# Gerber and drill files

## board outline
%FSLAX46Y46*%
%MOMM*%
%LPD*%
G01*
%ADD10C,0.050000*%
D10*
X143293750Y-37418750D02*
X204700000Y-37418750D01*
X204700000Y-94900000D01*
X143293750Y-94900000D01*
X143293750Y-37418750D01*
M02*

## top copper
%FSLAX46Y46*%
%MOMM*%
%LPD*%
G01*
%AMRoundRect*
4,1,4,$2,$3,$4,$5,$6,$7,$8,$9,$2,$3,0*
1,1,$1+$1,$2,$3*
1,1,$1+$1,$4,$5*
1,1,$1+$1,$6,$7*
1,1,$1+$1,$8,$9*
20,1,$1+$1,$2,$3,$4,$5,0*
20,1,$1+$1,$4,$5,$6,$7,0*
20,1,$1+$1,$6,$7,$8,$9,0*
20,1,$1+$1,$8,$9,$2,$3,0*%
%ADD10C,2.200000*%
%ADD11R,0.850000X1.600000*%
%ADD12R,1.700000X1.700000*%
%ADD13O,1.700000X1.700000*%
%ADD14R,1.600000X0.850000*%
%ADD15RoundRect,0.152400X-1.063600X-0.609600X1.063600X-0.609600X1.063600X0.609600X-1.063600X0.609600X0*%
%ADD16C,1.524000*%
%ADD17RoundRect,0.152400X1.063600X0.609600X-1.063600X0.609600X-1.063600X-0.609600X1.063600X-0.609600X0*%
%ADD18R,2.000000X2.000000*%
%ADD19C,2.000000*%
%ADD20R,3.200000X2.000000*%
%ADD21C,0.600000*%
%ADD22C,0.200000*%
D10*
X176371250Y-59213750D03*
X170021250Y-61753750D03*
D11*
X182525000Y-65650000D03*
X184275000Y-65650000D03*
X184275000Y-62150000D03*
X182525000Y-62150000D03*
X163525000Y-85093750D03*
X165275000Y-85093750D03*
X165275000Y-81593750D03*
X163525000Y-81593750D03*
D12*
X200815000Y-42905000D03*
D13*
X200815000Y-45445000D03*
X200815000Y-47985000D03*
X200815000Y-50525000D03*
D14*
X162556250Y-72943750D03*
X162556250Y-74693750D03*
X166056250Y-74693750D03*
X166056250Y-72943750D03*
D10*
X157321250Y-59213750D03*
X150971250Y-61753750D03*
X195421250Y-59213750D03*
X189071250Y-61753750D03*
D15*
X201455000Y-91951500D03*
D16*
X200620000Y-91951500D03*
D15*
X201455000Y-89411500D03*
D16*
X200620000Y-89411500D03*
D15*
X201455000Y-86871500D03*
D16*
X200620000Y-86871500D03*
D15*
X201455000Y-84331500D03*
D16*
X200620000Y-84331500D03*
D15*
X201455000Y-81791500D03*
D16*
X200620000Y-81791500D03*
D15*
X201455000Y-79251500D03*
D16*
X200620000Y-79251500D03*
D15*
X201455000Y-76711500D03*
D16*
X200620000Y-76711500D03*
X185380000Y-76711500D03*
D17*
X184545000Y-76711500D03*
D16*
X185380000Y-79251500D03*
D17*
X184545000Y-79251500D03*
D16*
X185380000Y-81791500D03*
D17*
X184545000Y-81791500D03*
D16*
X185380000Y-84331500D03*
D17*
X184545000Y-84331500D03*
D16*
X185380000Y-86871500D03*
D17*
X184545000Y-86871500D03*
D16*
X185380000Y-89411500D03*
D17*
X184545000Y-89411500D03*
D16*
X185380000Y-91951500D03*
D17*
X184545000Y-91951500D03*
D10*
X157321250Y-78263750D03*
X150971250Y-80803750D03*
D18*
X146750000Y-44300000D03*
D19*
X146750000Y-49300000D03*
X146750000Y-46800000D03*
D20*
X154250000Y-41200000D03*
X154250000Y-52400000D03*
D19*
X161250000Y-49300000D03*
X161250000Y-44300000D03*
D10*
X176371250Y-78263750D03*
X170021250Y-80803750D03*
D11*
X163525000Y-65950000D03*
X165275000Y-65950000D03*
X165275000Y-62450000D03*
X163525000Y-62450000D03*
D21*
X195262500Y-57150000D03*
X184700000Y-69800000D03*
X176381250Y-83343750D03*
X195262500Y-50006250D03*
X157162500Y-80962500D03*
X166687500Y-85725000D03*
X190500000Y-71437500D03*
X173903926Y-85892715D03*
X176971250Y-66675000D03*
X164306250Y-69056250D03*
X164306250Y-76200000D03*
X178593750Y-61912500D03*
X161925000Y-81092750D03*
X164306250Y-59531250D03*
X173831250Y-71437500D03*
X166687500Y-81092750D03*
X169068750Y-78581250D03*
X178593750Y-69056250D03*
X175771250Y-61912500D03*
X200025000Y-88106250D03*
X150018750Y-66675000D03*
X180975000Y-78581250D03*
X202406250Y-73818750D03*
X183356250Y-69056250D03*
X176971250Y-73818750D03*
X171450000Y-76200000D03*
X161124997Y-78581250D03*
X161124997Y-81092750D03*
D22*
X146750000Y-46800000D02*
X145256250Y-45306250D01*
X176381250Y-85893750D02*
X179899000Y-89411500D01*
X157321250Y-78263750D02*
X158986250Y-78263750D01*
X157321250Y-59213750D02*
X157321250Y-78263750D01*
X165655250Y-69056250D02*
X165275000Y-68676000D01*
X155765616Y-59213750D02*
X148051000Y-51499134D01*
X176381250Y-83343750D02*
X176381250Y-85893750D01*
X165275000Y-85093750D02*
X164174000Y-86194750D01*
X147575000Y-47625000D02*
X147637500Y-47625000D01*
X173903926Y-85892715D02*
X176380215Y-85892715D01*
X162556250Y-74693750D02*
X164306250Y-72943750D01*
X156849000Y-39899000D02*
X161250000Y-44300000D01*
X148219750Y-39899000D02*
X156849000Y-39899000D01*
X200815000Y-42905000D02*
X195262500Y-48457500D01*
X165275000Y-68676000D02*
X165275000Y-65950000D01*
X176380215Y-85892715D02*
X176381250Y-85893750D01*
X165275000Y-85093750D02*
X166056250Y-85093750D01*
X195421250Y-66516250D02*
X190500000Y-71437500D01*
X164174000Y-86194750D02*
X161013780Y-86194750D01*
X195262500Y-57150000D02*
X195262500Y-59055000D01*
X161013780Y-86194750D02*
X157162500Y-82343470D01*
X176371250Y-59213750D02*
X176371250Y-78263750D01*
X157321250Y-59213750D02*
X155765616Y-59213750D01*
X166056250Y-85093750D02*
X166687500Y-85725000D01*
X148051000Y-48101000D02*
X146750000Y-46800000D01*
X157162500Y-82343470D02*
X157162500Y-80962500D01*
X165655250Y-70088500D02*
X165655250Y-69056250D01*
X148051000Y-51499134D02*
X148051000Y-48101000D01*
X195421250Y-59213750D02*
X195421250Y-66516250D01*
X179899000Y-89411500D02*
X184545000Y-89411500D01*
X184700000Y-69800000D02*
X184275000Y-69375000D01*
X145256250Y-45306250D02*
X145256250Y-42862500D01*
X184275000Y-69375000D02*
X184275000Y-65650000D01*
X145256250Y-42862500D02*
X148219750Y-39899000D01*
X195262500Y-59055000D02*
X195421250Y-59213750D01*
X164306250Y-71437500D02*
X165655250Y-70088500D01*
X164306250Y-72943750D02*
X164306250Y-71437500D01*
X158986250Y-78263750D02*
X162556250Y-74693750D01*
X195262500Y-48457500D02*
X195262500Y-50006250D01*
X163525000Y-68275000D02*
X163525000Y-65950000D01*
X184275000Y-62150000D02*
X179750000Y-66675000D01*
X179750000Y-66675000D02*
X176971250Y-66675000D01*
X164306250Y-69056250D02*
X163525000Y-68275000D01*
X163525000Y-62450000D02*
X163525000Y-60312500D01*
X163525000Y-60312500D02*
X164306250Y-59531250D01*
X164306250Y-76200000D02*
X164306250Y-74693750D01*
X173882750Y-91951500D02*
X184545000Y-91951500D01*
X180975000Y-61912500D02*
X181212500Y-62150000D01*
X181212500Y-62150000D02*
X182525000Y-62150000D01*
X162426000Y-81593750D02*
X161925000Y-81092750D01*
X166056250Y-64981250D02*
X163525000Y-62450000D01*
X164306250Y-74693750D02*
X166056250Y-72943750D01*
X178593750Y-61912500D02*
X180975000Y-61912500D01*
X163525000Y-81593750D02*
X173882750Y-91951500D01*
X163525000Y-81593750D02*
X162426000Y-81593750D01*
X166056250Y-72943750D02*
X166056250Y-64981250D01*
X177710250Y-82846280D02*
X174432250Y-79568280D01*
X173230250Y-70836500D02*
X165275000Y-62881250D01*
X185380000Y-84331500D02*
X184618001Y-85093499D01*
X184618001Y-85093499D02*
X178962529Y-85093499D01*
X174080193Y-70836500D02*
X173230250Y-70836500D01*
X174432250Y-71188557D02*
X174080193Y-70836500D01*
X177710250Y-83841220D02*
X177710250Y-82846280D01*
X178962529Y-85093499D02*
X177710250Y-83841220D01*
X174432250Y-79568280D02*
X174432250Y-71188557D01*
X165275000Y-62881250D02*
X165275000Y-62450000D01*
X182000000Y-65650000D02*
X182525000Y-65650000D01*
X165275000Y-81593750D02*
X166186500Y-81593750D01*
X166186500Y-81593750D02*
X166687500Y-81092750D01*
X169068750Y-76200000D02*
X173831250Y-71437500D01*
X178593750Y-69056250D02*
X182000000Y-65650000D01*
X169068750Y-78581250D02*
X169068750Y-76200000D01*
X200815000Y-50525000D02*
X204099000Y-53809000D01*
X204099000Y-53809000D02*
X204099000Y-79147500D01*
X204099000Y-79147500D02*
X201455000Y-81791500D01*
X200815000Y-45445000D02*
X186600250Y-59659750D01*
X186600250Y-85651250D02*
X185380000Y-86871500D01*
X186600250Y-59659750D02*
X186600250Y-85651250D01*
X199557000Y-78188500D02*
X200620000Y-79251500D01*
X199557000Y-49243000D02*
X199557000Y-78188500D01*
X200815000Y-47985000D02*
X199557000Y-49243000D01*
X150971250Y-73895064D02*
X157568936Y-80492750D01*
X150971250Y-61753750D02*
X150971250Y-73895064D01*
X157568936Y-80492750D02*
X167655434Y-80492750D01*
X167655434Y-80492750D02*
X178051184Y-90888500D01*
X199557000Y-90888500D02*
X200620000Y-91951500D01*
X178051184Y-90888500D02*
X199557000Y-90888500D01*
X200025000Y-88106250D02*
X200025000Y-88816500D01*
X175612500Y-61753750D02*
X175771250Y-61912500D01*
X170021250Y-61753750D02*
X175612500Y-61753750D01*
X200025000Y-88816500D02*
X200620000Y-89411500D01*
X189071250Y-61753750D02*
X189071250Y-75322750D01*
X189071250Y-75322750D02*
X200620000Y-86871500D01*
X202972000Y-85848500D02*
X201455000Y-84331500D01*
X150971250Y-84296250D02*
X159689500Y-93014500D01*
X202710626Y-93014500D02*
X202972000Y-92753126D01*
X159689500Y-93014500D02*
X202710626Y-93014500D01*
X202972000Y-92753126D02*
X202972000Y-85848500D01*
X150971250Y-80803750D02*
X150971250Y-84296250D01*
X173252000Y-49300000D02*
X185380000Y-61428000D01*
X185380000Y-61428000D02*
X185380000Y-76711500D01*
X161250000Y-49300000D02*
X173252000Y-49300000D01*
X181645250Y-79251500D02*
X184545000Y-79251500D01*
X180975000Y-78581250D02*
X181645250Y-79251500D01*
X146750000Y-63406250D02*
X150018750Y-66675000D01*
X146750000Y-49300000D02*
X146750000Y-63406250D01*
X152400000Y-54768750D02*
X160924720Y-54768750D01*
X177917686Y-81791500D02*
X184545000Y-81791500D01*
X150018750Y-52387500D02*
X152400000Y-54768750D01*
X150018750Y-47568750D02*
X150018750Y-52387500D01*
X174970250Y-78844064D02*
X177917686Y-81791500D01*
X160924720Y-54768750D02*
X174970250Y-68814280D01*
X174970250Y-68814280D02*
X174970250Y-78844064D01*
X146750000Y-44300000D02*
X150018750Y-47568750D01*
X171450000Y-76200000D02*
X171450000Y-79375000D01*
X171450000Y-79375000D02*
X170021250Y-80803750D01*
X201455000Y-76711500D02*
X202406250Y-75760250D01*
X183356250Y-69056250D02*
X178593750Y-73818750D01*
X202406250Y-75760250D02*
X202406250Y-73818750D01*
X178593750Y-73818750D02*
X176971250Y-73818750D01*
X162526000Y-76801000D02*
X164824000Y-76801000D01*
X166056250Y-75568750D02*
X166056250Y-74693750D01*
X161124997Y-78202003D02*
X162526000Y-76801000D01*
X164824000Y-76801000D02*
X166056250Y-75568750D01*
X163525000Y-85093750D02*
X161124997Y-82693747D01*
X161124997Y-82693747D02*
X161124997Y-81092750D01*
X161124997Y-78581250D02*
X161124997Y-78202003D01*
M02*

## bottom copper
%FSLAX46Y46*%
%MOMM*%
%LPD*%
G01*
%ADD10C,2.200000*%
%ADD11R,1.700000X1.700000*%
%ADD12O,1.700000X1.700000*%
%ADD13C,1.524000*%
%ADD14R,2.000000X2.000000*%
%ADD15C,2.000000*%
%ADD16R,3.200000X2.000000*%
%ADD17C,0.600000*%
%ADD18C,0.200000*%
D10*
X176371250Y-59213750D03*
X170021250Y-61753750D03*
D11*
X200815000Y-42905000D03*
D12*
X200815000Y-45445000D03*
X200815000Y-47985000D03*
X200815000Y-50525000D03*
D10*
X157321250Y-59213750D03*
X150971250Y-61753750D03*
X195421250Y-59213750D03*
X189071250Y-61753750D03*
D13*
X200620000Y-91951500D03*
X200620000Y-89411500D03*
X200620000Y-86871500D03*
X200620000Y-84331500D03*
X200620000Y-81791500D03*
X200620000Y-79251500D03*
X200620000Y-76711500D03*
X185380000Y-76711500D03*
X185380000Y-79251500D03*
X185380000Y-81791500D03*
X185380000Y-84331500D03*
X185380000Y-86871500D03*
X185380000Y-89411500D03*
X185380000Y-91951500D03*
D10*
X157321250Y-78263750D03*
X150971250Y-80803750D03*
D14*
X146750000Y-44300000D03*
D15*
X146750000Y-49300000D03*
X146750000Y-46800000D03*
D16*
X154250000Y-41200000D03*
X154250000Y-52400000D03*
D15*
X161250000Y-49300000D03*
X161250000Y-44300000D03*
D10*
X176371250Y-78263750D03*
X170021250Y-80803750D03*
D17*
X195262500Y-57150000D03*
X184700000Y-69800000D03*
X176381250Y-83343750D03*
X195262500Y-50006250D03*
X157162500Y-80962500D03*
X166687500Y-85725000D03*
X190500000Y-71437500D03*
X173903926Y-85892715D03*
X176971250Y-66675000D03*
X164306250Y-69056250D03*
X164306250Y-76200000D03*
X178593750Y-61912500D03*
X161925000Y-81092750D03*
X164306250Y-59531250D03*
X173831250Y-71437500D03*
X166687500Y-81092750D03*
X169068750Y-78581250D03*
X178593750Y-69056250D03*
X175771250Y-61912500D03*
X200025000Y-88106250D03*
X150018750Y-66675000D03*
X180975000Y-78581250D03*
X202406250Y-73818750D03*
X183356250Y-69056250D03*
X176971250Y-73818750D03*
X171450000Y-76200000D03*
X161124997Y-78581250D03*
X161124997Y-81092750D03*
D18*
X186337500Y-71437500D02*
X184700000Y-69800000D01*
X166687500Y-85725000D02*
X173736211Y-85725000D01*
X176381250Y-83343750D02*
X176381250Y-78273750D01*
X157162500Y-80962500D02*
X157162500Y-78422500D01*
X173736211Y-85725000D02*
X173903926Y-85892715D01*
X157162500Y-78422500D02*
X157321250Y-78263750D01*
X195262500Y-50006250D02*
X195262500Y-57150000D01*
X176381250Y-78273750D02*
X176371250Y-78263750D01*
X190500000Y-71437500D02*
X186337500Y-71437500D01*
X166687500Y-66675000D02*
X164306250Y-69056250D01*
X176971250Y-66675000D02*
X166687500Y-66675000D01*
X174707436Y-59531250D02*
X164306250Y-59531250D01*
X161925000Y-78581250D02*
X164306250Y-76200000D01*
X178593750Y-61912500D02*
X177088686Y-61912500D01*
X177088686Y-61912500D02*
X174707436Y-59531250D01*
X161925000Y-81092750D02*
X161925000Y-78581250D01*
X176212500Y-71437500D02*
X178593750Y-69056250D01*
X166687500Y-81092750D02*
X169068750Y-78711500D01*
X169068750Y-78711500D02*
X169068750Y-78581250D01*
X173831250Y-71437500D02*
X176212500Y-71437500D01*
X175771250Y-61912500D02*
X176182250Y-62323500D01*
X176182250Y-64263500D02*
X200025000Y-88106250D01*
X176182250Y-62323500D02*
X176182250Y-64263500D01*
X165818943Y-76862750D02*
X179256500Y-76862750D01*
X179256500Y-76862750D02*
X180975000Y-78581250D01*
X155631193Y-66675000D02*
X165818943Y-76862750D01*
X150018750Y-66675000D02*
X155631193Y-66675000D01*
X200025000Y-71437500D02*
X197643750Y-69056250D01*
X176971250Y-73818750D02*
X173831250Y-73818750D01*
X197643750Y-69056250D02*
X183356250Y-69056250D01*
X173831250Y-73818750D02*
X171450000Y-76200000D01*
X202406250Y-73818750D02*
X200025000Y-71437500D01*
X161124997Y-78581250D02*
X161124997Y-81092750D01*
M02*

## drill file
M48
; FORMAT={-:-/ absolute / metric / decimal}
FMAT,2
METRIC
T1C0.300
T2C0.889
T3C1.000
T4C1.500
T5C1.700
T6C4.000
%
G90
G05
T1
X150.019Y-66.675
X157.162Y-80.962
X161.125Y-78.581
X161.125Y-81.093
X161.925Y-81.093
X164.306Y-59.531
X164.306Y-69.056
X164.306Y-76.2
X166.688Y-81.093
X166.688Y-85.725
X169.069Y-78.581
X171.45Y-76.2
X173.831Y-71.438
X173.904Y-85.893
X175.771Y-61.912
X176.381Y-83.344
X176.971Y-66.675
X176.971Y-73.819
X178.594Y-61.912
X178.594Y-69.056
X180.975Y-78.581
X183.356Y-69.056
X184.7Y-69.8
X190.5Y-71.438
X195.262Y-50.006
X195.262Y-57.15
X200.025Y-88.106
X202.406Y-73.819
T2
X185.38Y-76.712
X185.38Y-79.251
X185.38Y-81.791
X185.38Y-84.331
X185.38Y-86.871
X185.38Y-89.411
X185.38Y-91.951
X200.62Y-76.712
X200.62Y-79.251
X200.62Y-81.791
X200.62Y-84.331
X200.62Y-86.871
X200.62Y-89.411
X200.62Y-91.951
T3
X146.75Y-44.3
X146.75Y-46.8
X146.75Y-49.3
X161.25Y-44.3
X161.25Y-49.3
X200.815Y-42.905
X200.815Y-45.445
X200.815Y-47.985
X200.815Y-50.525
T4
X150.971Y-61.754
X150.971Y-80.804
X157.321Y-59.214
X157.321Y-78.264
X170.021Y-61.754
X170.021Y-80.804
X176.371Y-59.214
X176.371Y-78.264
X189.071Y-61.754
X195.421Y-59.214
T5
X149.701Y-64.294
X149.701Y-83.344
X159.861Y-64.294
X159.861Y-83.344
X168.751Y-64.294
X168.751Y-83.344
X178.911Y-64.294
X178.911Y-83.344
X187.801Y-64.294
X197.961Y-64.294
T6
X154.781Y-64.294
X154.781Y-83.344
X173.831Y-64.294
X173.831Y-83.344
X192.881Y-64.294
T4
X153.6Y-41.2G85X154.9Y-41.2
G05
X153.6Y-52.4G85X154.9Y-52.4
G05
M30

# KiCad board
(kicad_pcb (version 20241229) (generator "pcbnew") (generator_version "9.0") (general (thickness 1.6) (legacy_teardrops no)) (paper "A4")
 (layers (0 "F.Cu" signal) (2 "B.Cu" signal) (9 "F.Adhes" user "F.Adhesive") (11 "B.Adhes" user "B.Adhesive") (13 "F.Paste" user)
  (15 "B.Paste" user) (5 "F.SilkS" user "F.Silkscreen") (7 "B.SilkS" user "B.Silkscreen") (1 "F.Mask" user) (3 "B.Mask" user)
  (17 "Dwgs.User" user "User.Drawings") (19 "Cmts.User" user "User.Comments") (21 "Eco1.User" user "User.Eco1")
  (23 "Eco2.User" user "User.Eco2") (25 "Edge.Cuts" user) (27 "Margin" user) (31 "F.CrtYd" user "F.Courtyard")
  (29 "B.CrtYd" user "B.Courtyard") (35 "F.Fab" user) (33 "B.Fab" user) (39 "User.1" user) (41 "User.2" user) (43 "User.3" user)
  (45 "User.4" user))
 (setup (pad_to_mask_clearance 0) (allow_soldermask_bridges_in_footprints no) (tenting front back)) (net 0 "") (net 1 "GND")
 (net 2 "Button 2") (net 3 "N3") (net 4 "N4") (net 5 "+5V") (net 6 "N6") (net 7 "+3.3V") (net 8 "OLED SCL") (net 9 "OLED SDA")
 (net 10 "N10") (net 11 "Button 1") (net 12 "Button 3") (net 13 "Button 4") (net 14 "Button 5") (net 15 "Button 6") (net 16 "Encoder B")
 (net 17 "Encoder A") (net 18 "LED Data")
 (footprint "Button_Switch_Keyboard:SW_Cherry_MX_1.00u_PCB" (layer "F.Cu") (at 176.37125 59.21375)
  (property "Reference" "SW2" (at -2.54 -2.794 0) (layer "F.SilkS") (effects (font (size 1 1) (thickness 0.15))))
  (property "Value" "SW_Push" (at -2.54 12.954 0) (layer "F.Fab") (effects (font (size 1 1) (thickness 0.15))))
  (pad "" np_thru_hole circle (at -7.62 5.08) (size 1.7 1.7) (drill 1.7) (layers "*.Cu" "*.Mask"))
  (pad "" np_thru_hole circle (at -2.54 5.08) (size 4 4) (drill 4) (layers "*.Cu" "*.Mask"))
  (pad "" np_thru_hole circle (at 2.54 5.08) (size 1.7 1.7) (drill 1.7) (layers "*.Cu" "*.Mask"))
  (pad "1" thru_hole circle (at 0 0) (size 2.2 2.2) (drill 1.5) (layers "*.Cu" "*.Mask") (remove_unused_layers no) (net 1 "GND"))
  (pad "2" thru_hole circle (at -6.35 2.54) (size 2.2 2.2) (drill 1.5) (layers "*.Cu" "*.Mask") (remove_unused_layers no) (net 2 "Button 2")))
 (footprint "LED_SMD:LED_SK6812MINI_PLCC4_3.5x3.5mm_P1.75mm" (layer "F.Cu") (at 183.4 63.9 90)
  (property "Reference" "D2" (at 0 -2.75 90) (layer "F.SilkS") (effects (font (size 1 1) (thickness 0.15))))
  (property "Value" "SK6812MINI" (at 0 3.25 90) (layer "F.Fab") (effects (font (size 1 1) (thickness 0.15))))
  (pad "1" smd rect (at -1.75 -0.875 90) (size 1.6 0.85) (layers "F.Cu" "F.Mask" "F.Paste") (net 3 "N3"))
  (pad "2" smd rect (at -1.75 0.875 90) (size 1.6 0.85) (layers "F.Cu" "F.Mask" "F.Paste") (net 1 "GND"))
  (pad "3" smd rect (at 1.75 0.875 90) (size 1.6 0.85) (layers "F.Cu" "F.Mask" "F.Paste") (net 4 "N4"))
  (pad "4" smd rect (at 1.75 -0.875 90) (size 1.6 0.85) (layers "F.Cu" "F.Mask" "F.Paste") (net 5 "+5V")))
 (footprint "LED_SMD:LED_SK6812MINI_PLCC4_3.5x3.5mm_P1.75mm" (layer "F.Cu") (at 164.4 83.34375 90)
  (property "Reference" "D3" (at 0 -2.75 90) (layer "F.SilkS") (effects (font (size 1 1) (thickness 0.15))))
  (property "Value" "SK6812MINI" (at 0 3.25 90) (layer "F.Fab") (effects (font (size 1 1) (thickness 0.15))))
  (pad "1" smd rect (at -1.75 -0.875 90) (size 1.6 0.85) (layers "F.Cu" "F.Mask" "F.Paste") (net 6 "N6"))
  (pad "2" smd rect (at -1.75 0.875 90) (size 1.6 0.85) (layers "F.Cu" "F.Mask" "F.Paste") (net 1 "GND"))
  (pad "3" smd rect (at 1.75 0.875 90) (size 1.6 0.85) (layers "F.Cu" "F.Mask" "F.Paste") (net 3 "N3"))
  (pad "4" smd rect (at 1.75 -0.875 90) (size 1.6 0.85) (layers "F.Cu" "F.Mask" "F.Paste") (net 5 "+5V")))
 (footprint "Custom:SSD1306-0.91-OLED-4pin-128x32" (layer "F.Cu") (at 164.315 40.715)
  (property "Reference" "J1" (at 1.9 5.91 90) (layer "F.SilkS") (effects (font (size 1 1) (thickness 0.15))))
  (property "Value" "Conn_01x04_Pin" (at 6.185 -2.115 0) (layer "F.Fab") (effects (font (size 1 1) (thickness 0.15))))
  (pad "1" thru_hole rect (at 36.5 2.19) (size 1.7 1.7) (drill 1) (layers "*.Cu" "*.Mask") (remove_unused_layers no) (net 1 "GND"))
  (pad "2" thru_hole oval (at 36.5 4.73) (size 1.7 1.7) (drill 1) (layers "*.Cu" "*.Mask") (remove_unused_layers no) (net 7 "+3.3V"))
  (pad "3" thru_hole oval (at 36.5 7.27) (size 1.7 1.7) (drill 1) (layers "*.Cu" "*.Mask") (remove_unused_layers no) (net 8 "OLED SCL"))
  (pad "4" thru_hole oval (at 36.5 9.81) (size 1.7 1.7) (drill 1) (layers "*.Cu" "*.Mask") (remove_unused_layers no) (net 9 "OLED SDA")))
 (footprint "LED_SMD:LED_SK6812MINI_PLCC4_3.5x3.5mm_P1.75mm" (layer "F.Cu") (at 164.30625 73.81875)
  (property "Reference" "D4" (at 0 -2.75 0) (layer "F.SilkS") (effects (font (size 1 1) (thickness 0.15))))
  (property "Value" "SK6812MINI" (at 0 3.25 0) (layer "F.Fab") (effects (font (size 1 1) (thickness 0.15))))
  (pad "1" smd rect (at -1.75 -0.875) (size 1.6 0.85) (layers "F.Cu" "F.Mask" "F.Paste") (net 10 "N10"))
  (pad "2" smd rect (at -1.75 0.875) (size 1.6 0.85) (layers "F.Cu" "F.Mask" "F.Paste") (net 1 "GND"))
  (pad "3" smd rect (at 1.75 0.875) (size 1.6 0.85) (layers "F.Cu" "F.Mask" "F.Paste") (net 6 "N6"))
  (pad "4" smd rect (at 1.75 -0.875) (size 1.6 0.85) (layers "F.Cu" "F.Mask" "F.Paste") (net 5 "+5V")))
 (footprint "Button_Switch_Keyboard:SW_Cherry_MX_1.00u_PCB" (layer "F.Cu") (at 157.32125 59.21375)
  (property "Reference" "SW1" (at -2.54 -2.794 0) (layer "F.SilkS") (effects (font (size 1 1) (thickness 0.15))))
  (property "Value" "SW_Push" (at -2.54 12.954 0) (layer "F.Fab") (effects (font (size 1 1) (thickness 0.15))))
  (pad "" np_thru_hole circle (at -7.62 5.08) (size 1.7 1.7) (drill 1.7) (layers "*.Cu" "*.Mask"))
  (pad "" np_thru_hole circle (at -2.54 5.08) (size 4 4) (drill 4) (layers "*.Cu" "*.Mask"))
  (pad "" np_thru_hole circle (at 2.54 5.08) (size 1.7 1.7) (drill 1.7) (layers "*.Cu" "*.Mask"))
  (pad "1" thru_hole circle (at 0 0) (size 2.2 2.2) (drill 1.5) (layers "*.Cu" "*.Mask") (remove_unused_layers no) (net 1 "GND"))
  (pad "2" thru_hole circle (at -6.35 2.54) (size 2.2 2.2) (drill 1.5) (layers "*.Cu" "*.Mask") (remove_unused_layers no)
   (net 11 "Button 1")))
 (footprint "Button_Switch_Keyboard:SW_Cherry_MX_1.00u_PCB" (layer "F.Cu") (at 195.42125 59.21375)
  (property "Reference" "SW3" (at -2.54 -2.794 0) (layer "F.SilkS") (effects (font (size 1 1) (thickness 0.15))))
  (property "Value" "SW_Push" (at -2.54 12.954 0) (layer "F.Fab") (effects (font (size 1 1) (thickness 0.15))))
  (pad "" np_thru_hole circle (at -7.62 5.08) (size 1.7 1.7) (drill 1.7) (layers "*.Cu" "*.Mask"))
  (pad "" np_thru_hole circle (at -2.54 5.08) (size 4 4) (drill 4) (layers "*.Cu" "*.Mask"))
  (pad "" np_thru_hole circle (at 2.54 5.08) (size 1.7 1.7) (drill 1.7) (layers "*.Cu" "*.Mask"))
  (pad "1" thru_hole circle (at 0 0) (size 2.2 2.2) (drill 1.5) (layers "*.Cu" "*.Mask") (remove_unused_layers no) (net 1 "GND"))
  (pad "2" thru_hole circle (at -6.35 2.54) (size 2.2 2.2) (drill 1.5) (layers "*.Cu" "*.Mask") (remove_unused_layers no)
   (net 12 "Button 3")))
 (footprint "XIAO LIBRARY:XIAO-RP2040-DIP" (layer "F.Cu") (at 193 84.3315 180)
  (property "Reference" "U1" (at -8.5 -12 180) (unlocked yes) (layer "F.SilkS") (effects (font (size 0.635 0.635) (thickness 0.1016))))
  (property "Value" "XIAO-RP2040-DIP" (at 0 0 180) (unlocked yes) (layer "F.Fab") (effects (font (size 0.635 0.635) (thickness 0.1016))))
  (pad "1" smd roundrect (at -8.455 -7.62) (size 2.432 1.524) (layers "F.Cu" "F.Mask") (roundrect_rratio 0.1) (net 11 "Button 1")
   (thermal_bridge_angle 45))
  (pad "1" thru_hole circle (at -7.62 -7.62) (size 1.524 1.524) (drill 0.889) (layers "*.Cu" "*.Mask") (remove_unused_layers no)
   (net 11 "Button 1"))
  (pad "2" smd roundrect (at -8.455 -5.08) (size 2.432 1.524) (layers "F.Cu" "F.Mask") (roundrect_rratio 0.1) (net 2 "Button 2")
   (thermal_bridge_angle 45))
  (pad "2" thru_hole circle (at -7.62 -5.08) (size 1.524 1.524) (drill 0.889) (layers "*.Cu" "*.Mask") (remove_unused_layers no)
   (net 2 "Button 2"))
  (pad "3" smd roundrect (at -8.455 -2.54) (size 2.432 1.524) (layers "F.Cu" "F.Mask") (roundrect_rratio 0.1) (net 12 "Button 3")
   (thermal_bridge_angle 45))
  (pad "3" thru_hole circle (at -7.62 -2.54) (size 1.524 1.524) (drill 0.889) (layers "*.Cu" "*.Mask") (remove_unused_layers no)
   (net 12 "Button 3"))
  (pad "4" smd roundrect (at -8.455 0) (size 2.432 1.524) (layers "F.Cu" "F.Mask") (roundrect_rratio 0.1) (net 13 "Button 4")
   (thermal_bridge_angle 45))
  (pad "4" thru_hole circle (at -7.62 0) (size 1.524 1.524) (drill 0.889) (layers "*.Cu" "*.Mask") (remove_unused_layers no)
   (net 13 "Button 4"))
  (pad "5" smd roundrect (at -8.455 2.54) (size 2.432 1.524) (layers "F.Cu" "F.Mask") (roundrect_rratio 0.1) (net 9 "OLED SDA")
   (thermal_bridge_angle 45))
  (pad "5" thru_hole circle (at -7.62 2.54) (size 1.524 1.524) (drill 0.889) (layers "*.Cu" "*.Mask") (remove_unused_layers no)
   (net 9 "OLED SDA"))
  (pad "6" smd roundrect (at -8.455 5.08) (size 2.432 1.524) (layers "F.Cu" "F.Mask") (roundrect_rratio 0.1) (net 8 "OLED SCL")
   (thermal_bridge_angle 45))
  (pad "6" thru_hole circle (at -7.62 5.08) (size 1.524 1.524) (drill 0.889) (layers "*.Cu" "*.Mask") (remove_unused_layers no)
   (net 8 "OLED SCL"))
  (pad "7" smd roundrect (at -8.455 7.62) (size 2.432 1.524) (layers "F.Cu" "F.Mask") (roundrect_rratio 0.1) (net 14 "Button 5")
   (thermal_bridge_angle 45))
  (pad "7" thru_hole circle (at -7.62 7.62) (size 1.524 1.524) (drill 0.889) (layers "*.Cu" "*.Mask") (remove_unused_layers no)
   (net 14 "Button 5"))
  (pad "8" thru_hole circle (at 7.62 7.62 180) (size 1.524 1.524) (drill 0.889) (layers "*.Cu" "*.Mask") (remove_unused_layers no)
   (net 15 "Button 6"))
  (pad "8" smd roundrect (at 8.455 7.62 180) (size 2.432 1.524) (layers "F.Cu" "F.Mask") (roundrect_rratio 0.1) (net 15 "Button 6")
   (thermal_bridge_angle 45))
  (pad "9" thru_hole circle (at 7.62 5.08 180) (size 1.524 1.524) (drill 0.889) (layers "*.Cu" "*.Mask") (remove_unused_layers no)
   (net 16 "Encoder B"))
  (pad "9" smd roundrect (at 8.455 5.08 180) (size 2.432 1.524) (layers "F.Cu" "F.Mask") (roundrect_rratio 0.1) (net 16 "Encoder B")
   (thermal_bridge_angle 45))
  (pad "10" thru_hole circle (at 7.62 2.54 180) (size 1.524 1.524) (drill 0.889) (layers "*.Cu" "*.Mask") (remove_unused_layers no)
   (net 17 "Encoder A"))
  (pad "10" smd roundrect (at 8.455 2.54 180) (size 2.432 1.524) (layers "F.Cu" "F.Mask") (roundrect_rratio 0.1) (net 17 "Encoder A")
   (thermal_bridge_angle 45))
  (pad "11" thru_hole circle (at 7.62 0 180) (size 1.524 1.524) (drill 0.889) (layers "*.Cu" "*.Mask") (remove_unused_layers no)
   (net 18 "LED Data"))
  (pad "11" smd roundrect (at 8.455 0 180) (size 2.432 1.524) (layers "F.Cu" "F.Mask") (roundrect_rratio 0.1) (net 18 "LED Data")
   (thermal_bridge_angle 45))
  (pad "12" thru_hole circle (at 7.62 -2.54 180) (size 1.524 1.524) (drill 0.889) (layers "*.Cu" "*.Mask") (remove_unused_layers no)
   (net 7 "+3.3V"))
  (pad "12" smd roundrect (at 8.455 -2.54 180) (size 2.432 1.524) (layers "F.Cu" "F.Mask") (roundrect_rratio 0.1) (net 7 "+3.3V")
   (thermal_bridge_angle 45))
  (pad "13" thru_hole circle (at 7.62 -5.08 180) (size 1.524 1.524) (drill 0.889) (layers "*.Cu" "*.Mask") (remove_unused_layers no)
   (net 1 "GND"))
  (pad "13" smd roundrect (at 8.455 -5.08 180) (size 2.432 1.524) (layers "F.Cu" "F.Mask") (roundrect_rratio 0.1) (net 1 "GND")
   (thermal_bridge_angle 45))
  (pad "14" thru_hole circle (at 7.62 -7.62 180) (size 1.524 1.524) (drill 0.889) (layers "*.Cu" "*.Mask") (remove_unused_layers no)
   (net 5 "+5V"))
  (pad "14" smd roundrect (at 8.455 -7.62 180) (size 2.432 1.524) (layers "F.Cu" "F.Mask") (roundrect_rratio 0.1) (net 5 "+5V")
   (thermal_bridge_angle 45)))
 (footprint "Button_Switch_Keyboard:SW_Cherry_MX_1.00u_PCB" (layer "F.Cu") (at 157.32125 78.26375)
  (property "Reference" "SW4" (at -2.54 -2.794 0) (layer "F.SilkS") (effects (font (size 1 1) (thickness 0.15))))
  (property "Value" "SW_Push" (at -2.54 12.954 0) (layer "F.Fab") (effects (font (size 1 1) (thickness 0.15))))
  (pad "" np_thru_hole circle (at -7.62 5.08) (size 1.7 1.7) (drill 1.7) (layers "*.Cu" "*.Mask"))
  (pad "" np_thru_hole circle (at -2.54 5.08) (size 4 4) (drill 4) (layers "*.Cu" "*.Mask"))
  (pad "" np_thru_hole circle (at 2.54 5.08) (size 1.7 1.7) (drill 1.7) (layers "*.Cu" "*.Mask"))
  (pad "1" thru_hole circle (at 0 0) (size 2.2 2.2) (drill 1.5) (layers "*.Cu" "*.Mask") (remove_unused_layers no) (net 1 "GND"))
  (pad "2" thru_hole circle (at -6.35 2.54) (size 2.2 2.2) (drill 1.5) (layers "*.Cu" "*.Mask") (remove_unused_layers no)
   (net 13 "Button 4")))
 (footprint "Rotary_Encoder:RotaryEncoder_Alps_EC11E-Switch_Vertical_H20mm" (layer "F.Cu") (at 146.75 44.3)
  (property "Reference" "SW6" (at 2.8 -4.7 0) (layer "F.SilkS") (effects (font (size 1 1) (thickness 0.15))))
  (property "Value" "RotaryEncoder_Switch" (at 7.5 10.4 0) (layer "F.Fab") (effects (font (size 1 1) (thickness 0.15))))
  (pad "A" thru_hole rect (at 0 0) (size 2 2) (drill 1) (layers "*.Cu" "*.Mask") (remove_unused_layers no) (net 17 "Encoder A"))
  (pad "B" thru_hole circle (at 0 5) (size 2 2) (drill 1) (layers "*.Cu" "*.Mask") (remove_unused_layers no) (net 16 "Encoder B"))
  (pad "C" thru_hole circle (at 0 2.5) (size 2 2) (drill 1) (layers "*.Cu" "*.Mask") (remove_unused_layers no) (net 1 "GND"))
  (pad "MP" thru_hole rect (at 7.5 -3.1) (size 3.2 2) (drill oval 2.8 1.5) (layers "*.Cu" "*.Mask") (remove_unused_layers no))
  (pad "MP" thru_hole rect (at 7.5 8.1) (size 3.2 2) (drill oval 2.8 1.5) (layers "*.Cu" "*.Mask") (remove_unused_layers no))
  (pad "S1" thru_hole circle (at 14.5 5) (size 2 2) (drill 1) (layers "*.Cu" "*.Mask") (remove_unused_layers no) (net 15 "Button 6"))
  (pad "S2" thru_hole circle (at 14.5 0) (size 2 2) (drill 1) (layers "*.Cu" "*.Mask") (remove_unused_layers no) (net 1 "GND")))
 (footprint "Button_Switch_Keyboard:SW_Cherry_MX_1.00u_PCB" (layer "F.Cu") (at 176.37125 78.26375)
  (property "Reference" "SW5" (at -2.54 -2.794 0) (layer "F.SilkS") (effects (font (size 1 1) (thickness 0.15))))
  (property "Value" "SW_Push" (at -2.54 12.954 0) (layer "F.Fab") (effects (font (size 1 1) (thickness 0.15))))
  (pad "" np_thru_hole circle (at -7.62 5.08) (size 1.7 1.7) (drill 1.7) (layers "*.Cu" "*.Mask"))
  (pad "" np_thru_hole circle (at -2.54 5.08) (size 4 4) (drill 4) (layers "*.Cu" "*.Mask"))
  (pad "" np_thru_hole circle (at 2.54 5.08) (size 1.7 1.7) (drill 1.7) (layers "*.Cu" "*.Mask"))
  (pad "1" thru_hole circle (at 0 0) (size 2.2 2.2) (drill 1.5) (layers "*.Cu" "*.Mask") (remove_unused_layers no) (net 1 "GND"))
  (pad "2" thru_hole circle (at -6.35 2.54) (size 2.2 2.2) (drill 1.5) (layers "*.Cu" "*.Mask") (remove_unused_layers no)
   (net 14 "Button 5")))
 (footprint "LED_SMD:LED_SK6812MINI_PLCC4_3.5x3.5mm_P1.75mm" (layer "F.Cu") (at 164.4 64.2 90)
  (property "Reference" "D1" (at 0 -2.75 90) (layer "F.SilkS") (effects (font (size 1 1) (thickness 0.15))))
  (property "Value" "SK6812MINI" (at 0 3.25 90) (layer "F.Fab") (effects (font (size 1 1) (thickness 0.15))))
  (pad "1" smd rect (at -1.75 -0.875 90) (size 1.6 0.85) (layers "F.Cu" "F.Mask" "F.Paste") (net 4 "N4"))
  (pad "2" smd rect (at -1.75 0.875 90) (size 1.6 0.85) (layers "F.Cu" "F.Mask" "F.Paste") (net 1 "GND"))
  (pad "3" smd rect (at 1.75 0.875 90) (size 1.6 0.85) (layers "F.Cu" "F.Mask" "F.Paste") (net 18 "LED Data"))
  (pad "4" smd rect (at 1.75 -0.875 90) (size 1.6 0.85) (layers "F.Cu" "F.Mask" "F.Paste") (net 5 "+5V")))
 (gr_rect (start 143.29375 37.41875) (end 204.7 94.9) (stroke (width 0.05) (type default)) (fill no) (layer "Edge.Cuts"))
 (segment (start 146.75 46.8) (end 145.25625 45.30625) (width 0.2) (layer "F.Cu") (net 1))
 (segment (start 176.38125 85.89375) (end 179.899 89.4115) (width 0.2) (layer "F.Cu") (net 1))
 (segment (start 157.32125 78.26375) (end 158.98625 78.26375) (width 0.2) (layer "F.Cu") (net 1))
 (segment (start 157.32125 59.21375) (end 157.32125 78.26375) (width 0.2) (layer "F.Cu") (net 1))
 (segment (start 165.65525 69.05625) (end 165.275 68.676) (width 0.2) (layer "F.Cu") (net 1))
 (segment (start 155.765616 59.21375) (end 148.051 51.499134) (width 0.2) (layer "F.Cu") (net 1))
 (segment (start 176.38125 83.34375) (end 176.38125 85.89375) (width 0.2) (layer "F.Cu") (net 1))
 (segment (start 165.275 85.09375) (end 164.174 86.19475) (width 0.2) (layer "F.Cu") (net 1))
 (segment (start 147.575 47.625) (end 147.6375 47.625) (width 0.2) (layer "F.Cu") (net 1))
 (segment (start 173.903926 85.892715) (end 176.380215 85.892715) (width 0.2) (layer "F.Cu") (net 1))
 (segment (start 162.55625 74.69375) (end 164.30625 72.94375) (width 0.2) (layer "F.Cu") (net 1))
 (segment (start 156.849 39.899) (end 161.25 44.3) (width 0.2) (layer "F.Cu") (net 1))
 (segment (start 148.21975 39.899) (end 156.849 39.899) (width 0.2) (layer "F.Cu") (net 1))
 (segment (start 200.815 42.905) (end 195.2625 48.4575) (width 0.2) (layer "F.Cu") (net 1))
 (segment (start 165.275 68.676) (end 165.275 65.95) (width 0.2) (layer "F.Cu") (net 1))
 (segment (start 176.380215 85.892715) (end 176.38125 85.89375) (width 0.2) (layer "F.Cu") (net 1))
 (segment (start 165.275 85.09375) (end 166.05625 85.09375) (width 0.2) (layer "F.Cu") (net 1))
 (segment (start 195.42125 66.51625) (end 190.5 71.4375) (width 0.2) (layer "F.Cu") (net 1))
 (segment (start 164.174 86.19475) (end 161.01378 86.19475) (width 0.2) (layer "F.Cu") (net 1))
 (segment (start 195.2625 57.15) (end 195.2625 59.055) (width 0.2) (layer "F.Cu") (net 1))
 (segment (start 161.01378 86.19475) (end 157.1625 82.34347) (width 0.2) (layer "F.Cu") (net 1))
 (segment (start 176.37125 59.21375) (end 176.37125 78.26375) (width 0.2) (layer "F.Cu") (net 1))
 (segment (start 157.32125 59.21375) (end 155.765616 59.21375) (width 0.2) (layer "F.Cu") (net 1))
 (segment (start 166.05625 85.09375) (end 166.6875 85.725) (width 0.2) (layer "F.Cu") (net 1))
 (segment (start 148.051 48.101) (end 146.75 46.8) (width 0.2) (layer "F.Cu") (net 1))
 (segment (start 157.1625 82.34347) (end 157.1625 80.9625) (width 0.2) (layer "F.Cu") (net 1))
 (segment (start 165.65525 70.0885) (end 165.65525 69.05625) (width 0.2) (layer "F.Cu") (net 1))
 (segment (start 148.051 51.499134) (end 148.051 48.101) (width 0.2) (layer "F.Cu") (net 1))
 (segment (start 195.42125 59.21375) (end 195.42125 66.51625) (width 0.2) (layer "F.Cu") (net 1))
 (segment (start 179.899 89.4115) (end 184.545 89.4115) (width 0.2) (layer "F.Cu") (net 1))
 (segment (start 184.7 69.8) (end 184.275 69.375) (width 0.2) (layer "F.Cu") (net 1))
 (segment (start 145.25625 45.30625) (end 145.25625 42.8625) (width 0.2) (layer "F.Cu") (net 1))
 (segment (start 184.275 69.375) (end 184.275 65.65) (width 0.2) (layer "F.Cu") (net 1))
 (segment (start 145.25625 42.8625) (end 148.21975 39.899) (width 0.2) (layer "F.Cu") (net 1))
 (segment (start 195.2625 59.055) (end 195.42125 59.21375) (width 0.2) (layer "F.Cu") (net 1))
 (segment (start 164.30625 71.4375) (end 165.65525 70.0885) (width 0.2) (layer "F.Cu") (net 1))
 (segment (start 164.30625 72.94375) (end 164.30625 71.4375) (width 0.2) (layer "F.Cu") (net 1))
 (segment (start 158.98625 78.26375) (end 162.55625 74.69375) (width 0.2) (layer "F.Cu") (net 1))
 (segment (start 195.2625 48.4575) (end 195.2625 50.00625) (width 0.2) (layer "F.Cu") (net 1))
 (via (at 195.2625 57.15) (size 0.6) (drill 0.3) (layers "F.Cu" "B.Cu") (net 1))
 (via (at 184.7 69.8) (size 0.6) (drill 0.3) (layers "F.Cu" "B.Cu") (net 1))
 (via (at 176.38125 83.34375) (size 0.6) (drill 0.3) (layers "F.Cu" "B.Cu") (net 1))
 (via (at 195.2625 50.00625) (size 0.6) (drill 0.3) (layers "F.Cu" "B.Cu") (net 1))
 (via (at 157.1625 80.9625) (size 0.6) (drill 0.3) (layers "F.Cu" "B.Cu") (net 1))
 (via (at 166.6875 85.725) (size 0.6) (drill 0.3) (layers "F.Cu" "B.Cu") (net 1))
 (via (at 190.5 71.4375) (size 0.6) (drill 0.3) (layers "F.Cu" "B.Cu") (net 1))
 (via (at 173.903926 85.892715) (size 0.6) (drill 0.3) (layers "F.Cu" "B.Cu") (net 1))
 (segment (start 186.3375 71.4375) (end 184.7 69.8) (width 0.2) (layer "B.Cu") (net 1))
 (segment (start 166.6875 85.725) (end 173.736211 85.725) (width 0.2) (layer "B.Cu") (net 1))
 (segment (start 176.38125 83.34375) (end 176.38125 78.27375) (width 0.2) (layer "B.Cu") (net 1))
 (segment (start 157.1625 80.9625) (end 157.1625 78.4225) (width 0.2) (layer "B.Cu") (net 1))
 (segment (start 173.736211 85.725) (end 173.903926 85.892715) (width 0.2) (layer "B.Cu") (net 1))
 (segment (start 157.1625 78.4225) (end 157.32125 78.26375) (width 0.2) (layer "B.Cu") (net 1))
 (segment (start 195.2625 50.00625) (end 195.2625 57.15) (width 0.2) (layer "B.Cu") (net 1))
 (segment (start 176.38125 78.27375) (end 176.37125 78.26375) (width 0.2) (layer "B.Cu") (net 1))
 (segment (start 190.5 71.4375) (end 186.3375 71.4375) (width 0.2) (layer "B.Cu") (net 1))
 (segment (start 163.525 68.275) (end 163.525 65.95) (width 0.2) (layer "F.Cu") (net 4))
 (segment (start 184.275 62.15) (end 179.75 66.675) (width 0.2) (layer "F.Cu") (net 4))
 (segment (start 179.75 66.675) (end 176.97125 66.675) (width 0.2) (layer "F.Cu") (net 4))
 (segment (start 164.30625 69.05625) (end 163.525 68.275) (width 0.2) (layer "F.Cu") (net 4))
 (via (at 176.97125 66.675) (size 0.6) (drill 0.3) (layers "F.Cu" "B.Cu") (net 4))
 (via (at 164.30625 69.05625) (size 0.6) (drill 0.3) (layers "F.Cu" "B.Cu") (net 4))
 (segment (start 166.6875 66.675) (end 164.30625 69.05625) (width 0.2) (layer "B.Cu") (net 4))
 (segment (start 176.97125 66.675) (end 166.6875 66.675) (width 0.2) (layer "B.Cu") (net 4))
 (segment (start 163.525 62.45) (end 163.525 60.3125) (width 0.2) (layer "F.Cu") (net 5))
 (segment (start 163.525 60.3125) (end 164.30625 59.53125) (width 0.2) (layer "F.Cu") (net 5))
 (segment (start 164.30625 76.2) (end 164.30625 74.69375) (width 0.2) (layer "F.Cu") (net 5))
 (segment (start 173.88275 91.9515) (end 184.545 91.9515) (width 0.2) (layer "F.Cu") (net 5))
 (segment (start 180.975 61.9125) (end 181.2125 62.15) (width 0.2) (layer "F.Cu") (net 5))
 (segment (start 181.2125 62.15) (end 182.525 62.15) (width 0.2) (layer "F.Cu") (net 5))
 (segment (start 162.426 81.59375) (end 161.925 81.09275) (width 0.2) (layer "F.Cu") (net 5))
 (segment (start 166.05625 64.98125) (end 163.525 62.45) (width 0.2) (layer "F.Cu") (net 5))
 (segment (start 164.30625 74.69375) (end 166.05625 72.94375) (width 0.2) (layer "F.Cu") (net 5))
 (segment (start 178.59375 61.9125) (end 180.975 61.9125) (width 0.2) (layer "F.Cu") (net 5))
 (segment (start 163.525 81.59375) (end 173.88275 91.9515) (width 0.2) (layer "F.Cu") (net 5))
 (segment (start 163.525 81.59375) (end 162.426 81.59375) (width 0.2) (layer "F.Cu") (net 5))
 (segment (start 166.05625 72.94375) (end 166.05625 64.98125) (width 0.2) (layer "F.Cu") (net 5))
 (via (at 164.30625 76.2) (size 0.6) (drill 0.3) (layers "F.Cu" "B.Cu") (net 5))
 (via (at 178.59375 61.9125) (size 0.6) (drill 0.3) (layers "F.Cu" "B.Cu") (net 5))
 (via (at 161.925 81.09275) (size 0.6) (drill 0.3) (layers "F.Cu" "B.Cu") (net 5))
 (via (at 164.30625 59.53125) (size 0.6) (drill 0.3) (layers "F.Cu" "B.Cu") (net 5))
 (segment (start 174.707436 59.53125) (end 164.30625 59.53125) (width 0.2) (layer "B.Cu") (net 5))
 (segment (start 161.925 78.58125) (end 164.30625 76.2) (width 0.2) (layer "B.Cu") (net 5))
 (segment (start 178.59375 61.9125) (end 177.088686 61.9125) (width 0.2) (layer "B.Cu") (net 5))
 (segment (start 177.088686 61.9125) (end 174.707436 59.53125) (width 0.2) (layer "B.Cu") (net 5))
 (segment (start 161.925 81.09275) (end 161.925 78.58125) (width 0.2) (layer "B.Cu") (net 5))
 (segment (start 177.71025 82.84628) (end 174.43225 79.56828) (width 0.2) (layer "F.Cu") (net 18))
 (segment (start 173.23025 70.8365) (end 165.275 62.88125) (width 0.2) (layer "F.Cu") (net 18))
 (segment (start 185.38 84.3315) (end 184.618001 85.093499) (width 0.2) (layer "F.Cu") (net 18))
 (segment (start 184.618001 85.093499) (end 178.962529 85.093499) (width 0.2) (layer "F.Cu") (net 18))
 (segment (start 174.080193 70.8365) (end 173.23025 70.8365) (width 0.2) (layer "F.Cu") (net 18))
 (segment (start 174.43225 71.188557) (end 174.080193 70.8365) (width 0.2) (layer "F.Cu") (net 18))
 (segment (start 177.71025 83.84122) (end 177.71025 82.84628) (width 0.2) (layer "F.Cu") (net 18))
 (segment (start 178.962529 85.093499) (end 177.71025 83.84122) (width 0.2) (layer "F.Cu") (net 18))
 (segment (start 174.43225 79.56828) (end 174.43225 71.188557) (width 0.2) (layer "F.Cu") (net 18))
 (segment (start 165.275 62.88125) (end 165.275 62.45) (width 0.2) (layer "F.Cu") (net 18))
 (segment (start 182 65.65) (end 182.525 65.65) (width 0.2) (layer "F.Cu") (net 3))
 (segment (start 165.275 81.59375) (end 166.1865 81.59375) (width 0.2) (layer "F.Cu") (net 3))
 (segment (start 166.1865 81.59375) (end 166.6875 81.09275) (width 0.2) (layer "F.Cu") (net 3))
 (segment (start 169.06875 76.2) (end 173.83125 71.4375) (width 0.2) (layer "F.Cu") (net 3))
 (segment (start 178.59375 69.05625) (end 182 65.65) (width 0.2) (layer "F.Cu") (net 3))
 (segment (start 169.06875 78.58125) (end 169.06875 76.2) (width 0.2) (layer "F.Cu") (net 3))
 (via (at 173.83125 71.4375) (size 0.6) (drill 0.3) (layers "F.Cu" "B.Cu") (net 3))
 (via (at 166.6875 81.09275) (size 0.6) (drill 0.3) (layers "F.Cu" "B.Cu") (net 3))
 (via (at 169.06875 78.58125) (size 0.6) (drill 0.3) (layers "F.Cu" "B.Cu") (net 3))
 (via (at 178.59375 69.05625) (size 0.6) (drill 0.3) (layers "F.Cu" "B.Cu") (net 3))
 (segment (start 176.2125 71.4375) (end 178.59375 69.05625) (width 0.2) (layer "B.Cu") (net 3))
 (segment (start 166.6875 81.09275) (end 169.06875 78.7115) (width 0.2) (layer "B.Cu") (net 3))
 (segment (start 169.06875 78.7115) (end 169.06875 78.58125) (width 0.2) (layer "B.Cu") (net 3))
 (segment (start 173.83125 71.4375) (end 176.2125 71.4375) (width 0.2) (layer "B.Cu") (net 3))
 (segment (start 200.815 50.525) (end 204.099 53.809) (width 0.2) (layer "F.Cu") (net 9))
 (segment (start 204.099 53.809) (end 204.099 79.1475) (width 0.2) (layer "F.Cu") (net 9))
 (segment (start 204.099 79.1475) (end 201.455 81.7915) (width 0.2) (layer "F.Cu") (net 9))
 (segment (start 200.815 45.445) (end 186.60025 59.65975) (width 0.2) (layer "F.Cu") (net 7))
 (segment (start 186.60025 85.65125) (end 185.38 86.8715) (width 0.2) (layer "F.Cu") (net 7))
 (segment (start 186.60025 59.65975) (end 186.60025 85.65125) (width 0.2) (layer "F.Cu") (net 7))
 (segment (start 199.557 78.1885) (end 200.62 79.2515) (width 0.2) (layer "F.Cu") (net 8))
 (segment (start 199.557 49.243) (end 199.557 78.1885) (width 0.2) (layer "F.Cu") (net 8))
 (segment (start 200.815 47.985) (end 199.557 49.243) (width 0.2) (layer "F.Cu") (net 8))
 (segment (start 150.97125 73.895064) (end 157.568936 80.49275) (width 0.2) (layer "F.Cu") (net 11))
 (segment (start 150.97125 61.75375) (end 150.97125 73.895064) (width 0.2) (layer "F.Cu") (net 11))
 (segment (start 157.568936 80.49275) (end 167.655434 80.49275) (width 0.2) (layer "F.Cu") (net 11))
 (segment (start 167.655434 80.49275) (end 178.051184 90.8885) (width 0.2) (layer "F.Cu") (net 11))
 (segment (start 199.557 90.8885) (end 200.62 91.9515) (width 0.2) (layer "F.Cu") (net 11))
 (segment (start 178.051184 90.8885) (end 199.557 90.8885) (width 0.2) (layer "F.Cu") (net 11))
 (segment (start 200.025 88.10625) (end 200.025 88.8165) (width 0.2) (layer "F.Cu") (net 2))
 (segment (start 175.6125 61.75375) (end 175.77125 61.9125) (width 0.2) (layer "F.Cu") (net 2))
 (segment (start 170.02125 61.75375) (end 175.6125 61.75375) (width 0.2) (layer "F.Cu") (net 2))
 (segment (start 200.025 88.8165) (end 200.62 89.4115) (width 0.2) (layer "F.Cu") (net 2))
 (via (at 175.77125 61.9125) (size 0.6) (drill 0.3) (layers "F.Cu" "B.Cu") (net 2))
 (via (at 200.025 88.10625) (size 0.6) (drill 0.3) (layers "F.Cu" "B.Cu") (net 2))
 (segment (start 175.77125 61.9125) (end 176.18225 62.3235) (width 0.2) (layer "B.Cu") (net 2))
 (segment (start 176.18225 64.2635) (end 200.025 88.10625) (width 0.2) (layer "B.Cu") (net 2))
 (segment (start 176.18225 62.3235) (end 176.18225 64.2635) (width 0.2) (layer "B.Cu") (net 2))
 (segment (start 189.07125 61.75375) (end 189.07125 75.32275) (width 0.2) (layer "F.Cu") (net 12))
 (segment (start 189.07125 75.32275) (end 200.62 86.8715) (width 0.2) (layer "F.Cu") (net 12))
 (segment (start 202.972 85.8485) (end 201.455 84.3315) (width 0.2) (layer "F.Cu") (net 13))
 (segment (start 150.97125 84.29625) (end 159.6895 93.0145) (width 0.2) (layer "F.Cu") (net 13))
 (segment (start 202.710626 93.0145) (end 202.972 92.753126) (width 0.2) (layer "F.Cu") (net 13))
 (segment (start 159.6895 93.0145) (end 202.710626 93.0145) (width 0.2) (layer "F.Cu") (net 13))
 (segment (start 202.972 92.753126) (end 202.972 85.8485) (width 0.2) (layer "F.Cu") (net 13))
 (segment (start 150.97125 80.80375) (end 150.97125 84.29625) (width 0.2) (layer "F.Cu") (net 13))
 (segment (start 173.252 49.3) (end 185.38 61.428) (width 0.2) (layer "F.Cu") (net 15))
 (segment (start 185.38 61.428) (end 185.38 76.7115) (width 0.2) (layer "F.Cu") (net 15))
 (segment (start 161.25 49.3) (end 173.252 49.3) (width 0.2) (layer "F.Cu") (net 15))
 (segment (start 181.64525 79.2515) (end 184.545 79.2515) (width 0.2) (layer "F.Cu") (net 16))
 (segment (start 180.975 78.58125) (end 181.64525 79.2515) (width 0.2) (layer "F.Cu") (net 16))
 (segment (start 146.75 63.40625) (end 150.01875 66.675) (width 0.2) (layer "F.Cu") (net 16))
 (segment (start 146.75 49.3) (end 146.75 63.40625) (width 0.2) (layer "F.Cu") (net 16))
 (via (at 150.01875 66.675) (size 0.6) (drill 0.3) (layers "F.Cu" "B.Cu") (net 16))
 (via (at 180.975 78.58125) (size 0.6) (drill 0.3) (layers "F.Cu" "B.Cu") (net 16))
 (segment (start 165.818943 76.86275) (end 179.2565 76.86275) (width 0.2) (layer "B.Cu") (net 16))
 (segment (start 179.2565 76.86275) (end 180.975 78.58125) (width 0.2) (layer "B.Cu") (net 16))
 (segment (start 155.631193 66.675) (end 165.818943 76.86275) (width 0.2) (layer "B.Cu") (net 16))
 (segment (start 150.01875 66.675) (end 155.631193 66.675) (width 0.2) (layer "B.Cu") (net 16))
 (segment (start 152.4 54.76875) (end 160.92472 54.76875) (width 0.2) (layer "F.Cu") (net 17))
 (segment (start 177.917686 81.7915) (end 184.545 81.7915) (width 0.2) (layer "F.Cu") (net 17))
 (segment (start 150.01875 52.3875) (end 152.4 54.76875) (width 0.2) (layer "F.Cu") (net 17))
 (segment (start 150.01875 47.56875) (end 150.01875 52.3875) (width 0.2) (layer "F.Cu") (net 17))
 (segment (start 174.97025 78.844064) (end 177.917686 81.7915) (width 0.2) (layer "F.Cu") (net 17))
 (segment (start 160.92472 54.76875) (end 174.97025 68.81428) (width 0.2) (layer "F.Cu") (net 17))
 (segment (start 174.97025 68.81428) (end 174.97025 78.844064) (width 0.2) (layer "F.Cu") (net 17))
 (segment (start 146.75 44.3) (end 150.01875 47.56875) (width 0.2) (layer "F.Cu") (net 17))
 (segment (start 171.45 76.2) (end 171.45 79.375) (width 0.2) (layer "F.Cu") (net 14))
 (segment (start 171.45 79.375) (end 170.02125 80.80375) (width 0.2) (layer "F.Cu") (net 14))
 (segment (start 201.455 76.7115) (end 202.40625 75.76025) (width 0.2) (layer "F.Cu") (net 14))
 (segment (start 183.35625 69.05625) (end 178.59375 73.81875) (width 0.2) (layer "F.Cu") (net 14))
 (segment (start 202.40625 75.76025) (end 202.40625 73.81875) (width 0.2) (layer "F.Cu") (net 14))
 (segment (start 178.59375 73.81875) (end 176.97125 73.81875) (width 0.2) (layer "F.Cu") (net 14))
 (via (at 202.40625 73.81875) (size 0.6) (drill 0.3) (layers "F.Cu" "B.Cu") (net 14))
 (via (at 183.35625 69.05625) (size 0.6) (drill 0.3) (layers "F.Cu" "B.Cu") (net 14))
 (via (at 176.97125 73.81875) (size 0.6) (drill 0.3) (layers "F.Cu" "B.Cu") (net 14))
 (via (at 171.45 76.2) (size 0.6) (drill 0.3) (layers "F.Cu" "B.Cu") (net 14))
 (segment (start 200.025 71.4375) (end 197.64375 69.05625) (width 0.2) (layer "B.Cu") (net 14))
 (segment (start 176.97125 73.81875) (end 173.83125 73.81875) (width 0.2) (layer "B.Cu") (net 14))
 (segment (start 197.64375 69.05625) (end 183.35625 69.05625) (width 0.2) (layer "B.Cu") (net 14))
 (segment (start 173.83125 73.81875) (end 171.45 76.2) (width 0.2) (layer "B.Cu") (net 14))
 (segment (start 202.40625 73.81875) (end 200.025 71.4375) (width 0.2) (layer "B.Cu") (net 14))
 (segment (start 162.526 76.801) (end 164.824 76.801) (width 0.2) (layer "F.Cu") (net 6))
 (segment (start 166.05625 75.56875) (end 166.05625 74.69375) (width 0.2) (layer "F.Cu") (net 6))
 (segment (start 161.124997 78.202003) (end 162.526 76.801) (width 0.2) (layer "F.Cu") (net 6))
 (segment (start 164.824 76.801) (end 166.05625 75.56875) (width 0.2) (layer "F.Cu") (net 6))
 (segment (start 163.525 85.09375) (end 161.124997 82.693747) (width 0.2) (layer "F.Cu") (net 6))
 (segment (start 161.124997 82.693747) (end 161.124997 81.09275) (width 0.2) (layer "F.Cu") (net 6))
 (segment (start 161.124997 78.58125) (end 161.124997 78.202003) (width 0.2) (layer "F.Cu") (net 6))
 (via (at 161.124997 78.58125) (size 0.6) (drill 0.3) (layers "F.Cu" "B.Cu") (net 6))
 (via (at 161.124997 81.09275) (size 0.6) (drill 0.3) (layers "F.Cu" "B.Cu") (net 6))
 (segment (start 161.124997 78.58125) (end 161.124997 81.09275) (width 0.2) (layer "B.Cu") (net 6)))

